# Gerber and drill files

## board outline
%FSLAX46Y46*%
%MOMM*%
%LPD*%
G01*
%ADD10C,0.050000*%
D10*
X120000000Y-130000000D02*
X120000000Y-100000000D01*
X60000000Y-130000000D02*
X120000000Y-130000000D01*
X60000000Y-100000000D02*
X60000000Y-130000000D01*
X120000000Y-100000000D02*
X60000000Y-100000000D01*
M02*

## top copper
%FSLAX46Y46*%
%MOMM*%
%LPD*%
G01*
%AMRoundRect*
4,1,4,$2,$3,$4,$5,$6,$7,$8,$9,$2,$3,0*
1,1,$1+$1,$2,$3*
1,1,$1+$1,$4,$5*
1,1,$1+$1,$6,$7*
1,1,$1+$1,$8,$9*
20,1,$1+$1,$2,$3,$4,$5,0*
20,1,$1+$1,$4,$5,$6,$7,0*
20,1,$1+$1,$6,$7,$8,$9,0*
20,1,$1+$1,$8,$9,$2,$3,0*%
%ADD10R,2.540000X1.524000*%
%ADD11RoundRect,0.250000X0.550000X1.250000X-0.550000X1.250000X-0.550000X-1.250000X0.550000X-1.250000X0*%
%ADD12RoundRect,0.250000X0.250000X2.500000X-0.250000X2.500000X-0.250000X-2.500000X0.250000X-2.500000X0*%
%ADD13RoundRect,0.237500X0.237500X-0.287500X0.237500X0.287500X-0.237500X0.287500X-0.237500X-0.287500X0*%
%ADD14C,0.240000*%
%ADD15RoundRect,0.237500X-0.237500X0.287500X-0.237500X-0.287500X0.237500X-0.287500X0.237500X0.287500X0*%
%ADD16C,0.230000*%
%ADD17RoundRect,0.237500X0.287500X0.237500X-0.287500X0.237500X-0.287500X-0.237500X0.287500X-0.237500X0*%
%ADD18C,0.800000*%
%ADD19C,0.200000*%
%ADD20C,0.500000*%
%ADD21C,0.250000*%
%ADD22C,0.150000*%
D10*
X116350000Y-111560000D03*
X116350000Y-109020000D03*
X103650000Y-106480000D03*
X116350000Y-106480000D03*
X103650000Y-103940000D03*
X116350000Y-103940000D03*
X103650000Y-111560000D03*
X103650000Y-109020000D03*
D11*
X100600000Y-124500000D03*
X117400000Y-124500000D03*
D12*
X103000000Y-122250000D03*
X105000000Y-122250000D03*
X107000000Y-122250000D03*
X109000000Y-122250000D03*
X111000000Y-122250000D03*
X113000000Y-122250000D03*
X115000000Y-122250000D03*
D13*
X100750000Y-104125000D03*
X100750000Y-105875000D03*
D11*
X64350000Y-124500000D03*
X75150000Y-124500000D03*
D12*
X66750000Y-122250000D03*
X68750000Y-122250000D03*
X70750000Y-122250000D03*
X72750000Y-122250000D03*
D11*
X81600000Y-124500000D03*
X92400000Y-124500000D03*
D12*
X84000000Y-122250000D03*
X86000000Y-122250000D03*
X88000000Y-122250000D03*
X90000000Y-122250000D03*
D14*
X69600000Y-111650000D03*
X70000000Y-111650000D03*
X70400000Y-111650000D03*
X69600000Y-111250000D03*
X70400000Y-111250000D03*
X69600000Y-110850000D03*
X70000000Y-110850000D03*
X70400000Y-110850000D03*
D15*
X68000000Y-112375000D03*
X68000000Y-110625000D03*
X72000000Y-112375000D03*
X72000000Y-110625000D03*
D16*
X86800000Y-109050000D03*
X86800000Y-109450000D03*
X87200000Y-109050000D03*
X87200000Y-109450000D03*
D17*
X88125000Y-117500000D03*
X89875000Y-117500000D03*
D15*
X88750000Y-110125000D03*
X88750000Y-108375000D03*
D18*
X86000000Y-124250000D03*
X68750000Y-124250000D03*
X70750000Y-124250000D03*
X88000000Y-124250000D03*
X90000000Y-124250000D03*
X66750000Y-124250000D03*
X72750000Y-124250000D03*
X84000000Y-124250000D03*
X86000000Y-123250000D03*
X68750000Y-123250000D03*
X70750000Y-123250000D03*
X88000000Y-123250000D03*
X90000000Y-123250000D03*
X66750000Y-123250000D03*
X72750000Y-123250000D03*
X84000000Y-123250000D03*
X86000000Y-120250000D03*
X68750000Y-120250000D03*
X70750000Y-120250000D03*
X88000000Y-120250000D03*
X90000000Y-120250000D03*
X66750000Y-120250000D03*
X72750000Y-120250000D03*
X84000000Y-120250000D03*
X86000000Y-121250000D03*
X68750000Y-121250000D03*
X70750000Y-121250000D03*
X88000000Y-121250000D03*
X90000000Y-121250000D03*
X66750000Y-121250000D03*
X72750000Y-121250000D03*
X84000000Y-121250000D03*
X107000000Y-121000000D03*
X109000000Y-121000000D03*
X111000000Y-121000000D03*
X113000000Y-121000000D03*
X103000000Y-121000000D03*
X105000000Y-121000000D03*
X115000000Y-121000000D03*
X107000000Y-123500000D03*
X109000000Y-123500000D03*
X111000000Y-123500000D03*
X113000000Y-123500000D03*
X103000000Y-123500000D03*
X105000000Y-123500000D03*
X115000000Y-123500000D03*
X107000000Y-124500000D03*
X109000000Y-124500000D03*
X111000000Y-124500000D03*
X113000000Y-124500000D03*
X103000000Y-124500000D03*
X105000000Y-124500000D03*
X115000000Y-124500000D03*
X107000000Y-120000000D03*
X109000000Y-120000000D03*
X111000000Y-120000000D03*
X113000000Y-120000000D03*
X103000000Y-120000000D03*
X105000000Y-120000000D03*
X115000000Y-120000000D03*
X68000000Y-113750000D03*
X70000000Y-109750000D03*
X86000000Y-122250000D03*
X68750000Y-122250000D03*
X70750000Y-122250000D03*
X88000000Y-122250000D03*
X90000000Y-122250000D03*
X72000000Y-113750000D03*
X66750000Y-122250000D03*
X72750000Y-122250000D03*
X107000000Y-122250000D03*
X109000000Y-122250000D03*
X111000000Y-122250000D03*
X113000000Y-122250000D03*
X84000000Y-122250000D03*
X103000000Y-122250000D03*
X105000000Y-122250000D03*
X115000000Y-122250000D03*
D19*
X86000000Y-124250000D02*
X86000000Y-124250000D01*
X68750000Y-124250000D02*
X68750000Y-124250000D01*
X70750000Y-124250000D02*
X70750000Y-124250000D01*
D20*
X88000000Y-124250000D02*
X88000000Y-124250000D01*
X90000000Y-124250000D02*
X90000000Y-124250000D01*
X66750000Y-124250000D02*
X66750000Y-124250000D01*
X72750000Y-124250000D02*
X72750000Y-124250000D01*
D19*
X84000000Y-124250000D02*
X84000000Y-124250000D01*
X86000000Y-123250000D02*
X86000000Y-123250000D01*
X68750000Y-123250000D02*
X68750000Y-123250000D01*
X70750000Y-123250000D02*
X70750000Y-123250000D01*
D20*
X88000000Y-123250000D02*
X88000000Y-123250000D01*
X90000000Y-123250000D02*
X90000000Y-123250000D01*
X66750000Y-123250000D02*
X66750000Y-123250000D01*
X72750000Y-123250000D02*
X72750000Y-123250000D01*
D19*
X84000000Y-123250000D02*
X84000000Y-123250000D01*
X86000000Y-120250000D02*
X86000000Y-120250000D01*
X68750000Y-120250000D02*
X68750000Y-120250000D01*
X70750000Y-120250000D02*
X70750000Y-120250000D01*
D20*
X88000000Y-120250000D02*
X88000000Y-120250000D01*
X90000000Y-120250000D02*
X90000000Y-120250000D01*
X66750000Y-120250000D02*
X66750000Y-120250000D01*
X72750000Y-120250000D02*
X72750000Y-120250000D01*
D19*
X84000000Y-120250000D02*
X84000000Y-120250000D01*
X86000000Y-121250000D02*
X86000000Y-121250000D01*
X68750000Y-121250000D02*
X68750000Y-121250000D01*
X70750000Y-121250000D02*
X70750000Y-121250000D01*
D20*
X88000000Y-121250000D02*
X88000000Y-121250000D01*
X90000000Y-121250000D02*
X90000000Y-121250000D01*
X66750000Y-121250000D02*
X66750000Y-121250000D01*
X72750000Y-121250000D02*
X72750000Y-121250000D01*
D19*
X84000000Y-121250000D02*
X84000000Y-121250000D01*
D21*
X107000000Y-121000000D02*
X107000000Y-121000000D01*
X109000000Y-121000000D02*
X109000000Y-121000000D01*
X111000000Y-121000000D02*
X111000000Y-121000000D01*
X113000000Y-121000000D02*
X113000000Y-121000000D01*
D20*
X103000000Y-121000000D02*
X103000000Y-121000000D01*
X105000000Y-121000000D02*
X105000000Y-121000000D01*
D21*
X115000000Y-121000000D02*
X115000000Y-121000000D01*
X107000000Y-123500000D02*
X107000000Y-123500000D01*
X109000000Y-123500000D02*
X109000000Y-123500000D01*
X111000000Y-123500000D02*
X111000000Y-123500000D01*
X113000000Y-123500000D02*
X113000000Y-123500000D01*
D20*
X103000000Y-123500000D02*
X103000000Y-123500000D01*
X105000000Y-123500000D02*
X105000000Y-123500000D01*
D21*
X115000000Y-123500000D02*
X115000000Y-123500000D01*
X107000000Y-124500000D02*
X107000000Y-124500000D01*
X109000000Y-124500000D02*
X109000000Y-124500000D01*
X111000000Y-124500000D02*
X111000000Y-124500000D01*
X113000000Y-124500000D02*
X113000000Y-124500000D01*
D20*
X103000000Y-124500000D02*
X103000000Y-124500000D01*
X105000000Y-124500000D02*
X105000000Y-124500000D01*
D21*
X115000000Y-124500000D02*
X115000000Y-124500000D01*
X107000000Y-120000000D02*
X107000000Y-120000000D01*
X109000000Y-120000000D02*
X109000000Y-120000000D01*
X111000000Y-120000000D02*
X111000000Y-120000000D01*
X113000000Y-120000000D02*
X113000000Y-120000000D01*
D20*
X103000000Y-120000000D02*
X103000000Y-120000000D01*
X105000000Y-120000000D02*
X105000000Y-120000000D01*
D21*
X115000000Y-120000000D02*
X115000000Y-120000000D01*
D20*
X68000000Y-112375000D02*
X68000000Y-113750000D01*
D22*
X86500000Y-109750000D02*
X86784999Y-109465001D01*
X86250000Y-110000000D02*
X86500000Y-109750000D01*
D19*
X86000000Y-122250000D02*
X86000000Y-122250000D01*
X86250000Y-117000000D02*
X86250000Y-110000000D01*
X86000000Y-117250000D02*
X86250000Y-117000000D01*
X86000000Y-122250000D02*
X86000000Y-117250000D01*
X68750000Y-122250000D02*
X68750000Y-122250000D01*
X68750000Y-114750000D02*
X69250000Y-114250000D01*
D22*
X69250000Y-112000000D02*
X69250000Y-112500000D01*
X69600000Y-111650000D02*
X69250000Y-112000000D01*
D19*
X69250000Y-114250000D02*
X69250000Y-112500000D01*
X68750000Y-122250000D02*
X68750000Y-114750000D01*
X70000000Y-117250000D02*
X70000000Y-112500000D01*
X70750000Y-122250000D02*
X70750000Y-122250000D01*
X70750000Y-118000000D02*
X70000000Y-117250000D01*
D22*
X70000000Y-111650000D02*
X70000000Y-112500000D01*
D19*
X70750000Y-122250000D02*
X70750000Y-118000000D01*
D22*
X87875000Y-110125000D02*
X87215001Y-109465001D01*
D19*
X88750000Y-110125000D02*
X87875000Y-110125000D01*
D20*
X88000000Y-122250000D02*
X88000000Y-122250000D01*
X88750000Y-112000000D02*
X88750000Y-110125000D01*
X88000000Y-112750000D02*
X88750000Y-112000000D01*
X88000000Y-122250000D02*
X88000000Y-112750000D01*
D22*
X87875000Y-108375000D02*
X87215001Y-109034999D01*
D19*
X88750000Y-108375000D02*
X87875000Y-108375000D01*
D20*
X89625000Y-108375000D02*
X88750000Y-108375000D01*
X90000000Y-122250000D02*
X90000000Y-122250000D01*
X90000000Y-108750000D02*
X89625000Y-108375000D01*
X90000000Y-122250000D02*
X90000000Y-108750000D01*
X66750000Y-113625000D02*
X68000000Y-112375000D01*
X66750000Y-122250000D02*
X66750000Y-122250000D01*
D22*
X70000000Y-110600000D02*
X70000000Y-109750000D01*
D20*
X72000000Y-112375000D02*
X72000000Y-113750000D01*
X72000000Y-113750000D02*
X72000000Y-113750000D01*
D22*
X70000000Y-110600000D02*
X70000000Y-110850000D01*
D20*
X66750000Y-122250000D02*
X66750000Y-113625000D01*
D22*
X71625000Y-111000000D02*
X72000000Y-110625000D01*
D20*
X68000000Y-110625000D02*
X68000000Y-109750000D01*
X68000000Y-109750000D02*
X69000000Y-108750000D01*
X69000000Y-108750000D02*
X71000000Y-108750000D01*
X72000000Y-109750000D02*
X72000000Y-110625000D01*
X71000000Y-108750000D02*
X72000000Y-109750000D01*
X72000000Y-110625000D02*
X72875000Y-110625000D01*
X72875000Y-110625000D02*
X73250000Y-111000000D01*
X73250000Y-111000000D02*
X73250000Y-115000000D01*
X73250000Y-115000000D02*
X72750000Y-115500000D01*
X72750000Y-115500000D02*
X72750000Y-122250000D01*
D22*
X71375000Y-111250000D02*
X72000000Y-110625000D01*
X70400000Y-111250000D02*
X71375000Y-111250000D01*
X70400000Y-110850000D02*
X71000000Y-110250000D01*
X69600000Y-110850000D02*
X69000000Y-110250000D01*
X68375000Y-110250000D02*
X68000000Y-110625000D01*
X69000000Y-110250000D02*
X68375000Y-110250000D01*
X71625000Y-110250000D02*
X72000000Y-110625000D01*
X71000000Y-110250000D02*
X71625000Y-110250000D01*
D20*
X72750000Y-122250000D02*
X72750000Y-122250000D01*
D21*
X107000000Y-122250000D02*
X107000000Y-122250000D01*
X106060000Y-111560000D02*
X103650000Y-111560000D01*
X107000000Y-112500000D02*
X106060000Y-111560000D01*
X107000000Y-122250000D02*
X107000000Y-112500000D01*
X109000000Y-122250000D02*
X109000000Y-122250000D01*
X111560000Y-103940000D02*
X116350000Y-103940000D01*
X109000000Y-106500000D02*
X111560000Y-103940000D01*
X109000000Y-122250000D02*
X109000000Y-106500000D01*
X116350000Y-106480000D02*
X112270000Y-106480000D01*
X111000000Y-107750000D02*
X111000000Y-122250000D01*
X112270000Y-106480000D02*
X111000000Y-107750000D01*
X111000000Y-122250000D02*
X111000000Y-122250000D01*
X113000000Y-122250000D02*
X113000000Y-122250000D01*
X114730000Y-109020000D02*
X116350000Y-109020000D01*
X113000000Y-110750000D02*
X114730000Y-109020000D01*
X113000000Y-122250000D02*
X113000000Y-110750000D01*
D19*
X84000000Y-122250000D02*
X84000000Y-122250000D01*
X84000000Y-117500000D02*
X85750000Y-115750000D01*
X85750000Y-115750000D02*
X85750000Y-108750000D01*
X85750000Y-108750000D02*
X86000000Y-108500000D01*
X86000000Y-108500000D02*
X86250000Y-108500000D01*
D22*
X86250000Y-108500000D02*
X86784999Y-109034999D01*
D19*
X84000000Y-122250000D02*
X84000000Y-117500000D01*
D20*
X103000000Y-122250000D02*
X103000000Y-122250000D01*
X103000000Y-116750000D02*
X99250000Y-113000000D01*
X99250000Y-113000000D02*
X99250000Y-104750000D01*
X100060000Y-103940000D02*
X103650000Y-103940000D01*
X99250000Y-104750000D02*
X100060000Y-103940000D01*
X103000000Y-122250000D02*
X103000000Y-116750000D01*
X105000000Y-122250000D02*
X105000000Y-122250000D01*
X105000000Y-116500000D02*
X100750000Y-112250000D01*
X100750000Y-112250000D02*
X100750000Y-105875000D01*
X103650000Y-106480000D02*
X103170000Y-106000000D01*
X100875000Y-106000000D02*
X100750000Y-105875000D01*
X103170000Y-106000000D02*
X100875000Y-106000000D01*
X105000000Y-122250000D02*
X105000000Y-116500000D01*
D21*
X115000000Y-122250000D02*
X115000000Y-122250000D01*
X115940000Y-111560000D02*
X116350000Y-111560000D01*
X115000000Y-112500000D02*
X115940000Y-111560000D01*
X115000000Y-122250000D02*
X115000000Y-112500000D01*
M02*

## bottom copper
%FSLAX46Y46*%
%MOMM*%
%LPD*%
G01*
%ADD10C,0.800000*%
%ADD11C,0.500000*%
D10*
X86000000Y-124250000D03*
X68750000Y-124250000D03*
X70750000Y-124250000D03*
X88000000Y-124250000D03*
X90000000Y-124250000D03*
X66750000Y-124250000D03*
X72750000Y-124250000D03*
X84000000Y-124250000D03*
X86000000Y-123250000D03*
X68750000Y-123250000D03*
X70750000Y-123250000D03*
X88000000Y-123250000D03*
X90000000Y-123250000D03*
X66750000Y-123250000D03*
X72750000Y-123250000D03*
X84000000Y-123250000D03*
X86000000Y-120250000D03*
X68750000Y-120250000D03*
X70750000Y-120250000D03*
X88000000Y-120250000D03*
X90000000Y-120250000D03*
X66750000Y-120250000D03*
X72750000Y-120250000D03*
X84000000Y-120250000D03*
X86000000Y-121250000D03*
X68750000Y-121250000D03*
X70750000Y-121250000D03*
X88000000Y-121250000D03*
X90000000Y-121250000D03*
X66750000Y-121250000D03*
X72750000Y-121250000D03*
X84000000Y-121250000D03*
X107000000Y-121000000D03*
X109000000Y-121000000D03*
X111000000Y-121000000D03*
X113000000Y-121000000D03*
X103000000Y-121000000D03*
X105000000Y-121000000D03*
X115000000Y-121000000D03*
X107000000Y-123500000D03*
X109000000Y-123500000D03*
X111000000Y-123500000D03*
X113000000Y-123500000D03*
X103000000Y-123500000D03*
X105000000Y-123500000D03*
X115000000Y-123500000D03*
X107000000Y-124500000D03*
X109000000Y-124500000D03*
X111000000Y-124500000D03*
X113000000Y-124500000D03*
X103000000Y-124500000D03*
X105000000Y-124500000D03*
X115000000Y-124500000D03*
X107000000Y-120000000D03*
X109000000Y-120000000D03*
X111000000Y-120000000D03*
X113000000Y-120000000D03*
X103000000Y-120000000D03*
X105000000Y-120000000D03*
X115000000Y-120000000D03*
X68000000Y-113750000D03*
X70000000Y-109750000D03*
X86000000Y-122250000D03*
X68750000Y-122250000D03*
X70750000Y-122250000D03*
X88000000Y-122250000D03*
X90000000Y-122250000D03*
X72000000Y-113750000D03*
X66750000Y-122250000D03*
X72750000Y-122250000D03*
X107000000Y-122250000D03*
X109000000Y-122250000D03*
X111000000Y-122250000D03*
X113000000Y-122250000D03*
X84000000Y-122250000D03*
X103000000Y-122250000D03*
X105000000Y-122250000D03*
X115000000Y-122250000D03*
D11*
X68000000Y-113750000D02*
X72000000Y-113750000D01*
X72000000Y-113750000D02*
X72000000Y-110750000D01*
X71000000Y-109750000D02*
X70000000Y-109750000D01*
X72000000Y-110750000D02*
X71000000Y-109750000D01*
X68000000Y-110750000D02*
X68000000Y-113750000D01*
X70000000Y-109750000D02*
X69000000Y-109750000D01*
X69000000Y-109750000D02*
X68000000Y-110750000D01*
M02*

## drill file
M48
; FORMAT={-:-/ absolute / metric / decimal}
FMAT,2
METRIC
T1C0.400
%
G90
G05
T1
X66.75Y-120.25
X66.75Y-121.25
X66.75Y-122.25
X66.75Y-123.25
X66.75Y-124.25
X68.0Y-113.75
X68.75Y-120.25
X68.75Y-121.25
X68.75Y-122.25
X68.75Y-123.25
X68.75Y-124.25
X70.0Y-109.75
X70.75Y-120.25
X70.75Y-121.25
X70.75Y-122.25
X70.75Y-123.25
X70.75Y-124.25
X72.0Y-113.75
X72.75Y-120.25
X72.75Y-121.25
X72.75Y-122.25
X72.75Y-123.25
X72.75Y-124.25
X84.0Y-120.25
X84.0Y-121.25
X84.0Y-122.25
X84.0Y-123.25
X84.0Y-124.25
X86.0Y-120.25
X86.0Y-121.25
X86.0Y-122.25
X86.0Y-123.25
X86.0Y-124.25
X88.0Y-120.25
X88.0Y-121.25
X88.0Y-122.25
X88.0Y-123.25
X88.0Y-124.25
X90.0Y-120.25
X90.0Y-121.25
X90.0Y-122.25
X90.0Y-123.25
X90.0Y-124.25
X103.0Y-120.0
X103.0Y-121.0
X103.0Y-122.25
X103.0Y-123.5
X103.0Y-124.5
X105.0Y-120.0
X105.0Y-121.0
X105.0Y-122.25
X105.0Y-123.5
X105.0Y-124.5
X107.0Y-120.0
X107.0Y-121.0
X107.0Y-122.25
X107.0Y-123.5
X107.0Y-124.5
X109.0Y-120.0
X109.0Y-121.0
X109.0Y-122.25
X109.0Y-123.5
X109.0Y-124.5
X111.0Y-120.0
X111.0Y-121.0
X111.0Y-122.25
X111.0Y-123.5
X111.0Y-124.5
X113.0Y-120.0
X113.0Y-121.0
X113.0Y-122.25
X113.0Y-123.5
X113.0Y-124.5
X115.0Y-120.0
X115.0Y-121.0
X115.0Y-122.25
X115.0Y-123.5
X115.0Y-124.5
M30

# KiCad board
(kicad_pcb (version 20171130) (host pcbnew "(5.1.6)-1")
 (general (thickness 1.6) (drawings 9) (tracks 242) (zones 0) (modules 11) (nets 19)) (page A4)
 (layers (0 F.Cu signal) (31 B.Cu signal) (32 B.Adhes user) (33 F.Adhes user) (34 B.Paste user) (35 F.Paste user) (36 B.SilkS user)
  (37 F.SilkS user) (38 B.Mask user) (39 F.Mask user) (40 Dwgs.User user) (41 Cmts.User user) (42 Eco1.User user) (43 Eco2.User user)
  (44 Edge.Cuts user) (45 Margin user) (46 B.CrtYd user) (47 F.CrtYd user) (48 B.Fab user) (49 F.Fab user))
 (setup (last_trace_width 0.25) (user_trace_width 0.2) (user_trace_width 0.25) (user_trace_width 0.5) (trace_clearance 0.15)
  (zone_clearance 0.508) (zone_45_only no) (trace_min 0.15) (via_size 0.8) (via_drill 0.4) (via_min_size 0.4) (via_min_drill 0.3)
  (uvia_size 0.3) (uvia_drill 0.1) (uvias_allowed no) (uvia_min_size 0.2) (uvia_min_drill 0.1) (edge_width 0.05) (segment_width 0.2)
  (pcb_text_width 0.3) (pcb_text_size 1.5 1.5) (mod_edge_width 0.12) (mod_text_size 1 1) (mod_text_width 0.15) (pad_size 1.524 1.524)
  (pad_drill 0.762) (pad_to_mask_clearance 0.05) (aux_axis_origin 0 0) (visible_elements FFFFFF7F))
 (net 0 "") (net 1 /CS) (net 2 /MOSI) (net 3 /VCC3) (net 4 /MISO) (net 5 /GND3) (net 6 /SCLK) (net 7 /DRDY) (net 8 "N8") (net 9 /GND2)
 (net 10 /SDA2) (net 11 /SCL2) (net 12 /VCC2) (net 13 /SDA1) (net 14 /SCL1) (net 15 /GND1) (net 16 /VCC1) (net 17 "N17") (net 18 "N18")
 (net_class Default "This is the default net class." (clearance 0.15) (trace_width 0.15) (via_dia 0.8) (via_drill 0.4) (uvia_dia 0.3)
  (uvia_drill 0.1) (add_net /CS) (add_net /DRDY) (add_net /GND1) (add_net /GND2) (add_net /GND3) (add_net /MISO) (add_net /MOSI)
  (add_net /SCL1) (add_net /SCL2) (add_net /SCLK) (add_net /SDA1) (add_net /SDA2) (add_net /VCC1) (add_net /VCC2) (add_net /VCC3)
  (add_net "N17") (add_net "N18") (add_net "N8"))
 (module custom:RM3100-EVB (layer F.Cu) (at 110 107.75)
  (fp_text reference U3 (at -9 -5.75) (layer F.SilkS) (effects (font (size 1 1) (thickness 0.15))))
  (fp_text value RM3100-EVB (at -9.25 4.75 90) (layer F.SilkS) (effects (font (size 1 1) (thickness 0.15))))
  (pad 8 smd rect (at 6.35 3.81) (size 2.54 1.524) (layers F.Cu F.Paste F.Mask) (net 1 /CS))
  (pad 7 smd rect (at 6.35 1.27) (size 2.54 1.524) (layers F.Cu F.Paste F.Mask) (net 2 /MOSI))
  (pad 2 smd rect (at -6.35 -1.27) (size 2.54 1.524) (layers F.Cu F.Paste F.Mask) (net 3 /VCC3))
  (pad 6 smd rect (at 6.35 -1.27) (size 2.54 1.524) (layers F.Cu F.Paste F.Mask) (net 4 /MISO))
  (pad 1 smd rect (at -6.35 -3.81) (size 2.54 1.524) (layers F.Cu F.Paste F.Mask) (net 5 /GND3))
  (pad 5 smd rect (at 6.35 -3.81) (size 2.54 1.524) (layers F.Cu F.Paste F.Mask) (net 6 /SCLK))
  (pad 4 smd rect (at -6.35 3.81) (size 2.54 1.524) (layers F.Cu F.Paste F.Mask) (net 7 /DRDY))
  (pad 3 smd rect (at -6.35 1.27) (size 2.54 1.524) (layers F.Cu F.Paste F.Mask) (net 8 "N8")))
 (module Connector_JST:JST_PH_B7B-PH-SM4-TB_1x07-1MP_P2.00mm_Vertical (layer F.Cu) (at 109 122.75 180)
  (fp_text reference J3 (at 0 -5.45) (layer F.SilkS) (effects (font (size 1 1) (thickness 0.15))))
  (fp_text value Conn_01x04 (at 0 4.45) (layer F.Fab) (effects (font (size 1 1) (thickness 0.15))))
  (pad MP smd roundrect (at 8.4 -1.75 180) (size 1.6 3) (layers F.Cu F.Paste F.Mask) (roundrect_rratio 0.15625))
  (pad MP smd roundrect (at -8.4 -1.75 180) (size 1.6 3) (layers F.Cu F.Paste F.Mask) (roundrect_rratio 0.15625))
  (pad 7 smd roundrect (at 6 0.5 180) (size 1 5.5) (layers F.Cu F.Paste F.Mask) (roundrect_rratio 0.25) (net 5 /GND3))
  (pad 6 smd roundrect (at 4 0.5 180) (size 1 5.5) (layers F.Cu F.Paste F.Mask) (roundrect_rratio 0.25) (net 3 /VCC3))
  (pad 5 smd roundrect (at 2 0.5 180) (size 1 5.5) (layers F.Cu F.Paste F.Mask) (roundrect_rratio 0.25) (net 7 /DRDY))
  (pad 4 smd roundrect (at 0 0.5 180) (size 1 5.5) (layers F.Cu F.Paste F.Mask) (roundrect_rratio 0.25) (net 6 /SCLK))
  (pad 3 smd roundrect (at -2 0.5 180) (size 1 5.5) (layers F.Cu F.Paste F.Mask) (roundrect_rratio 0.25) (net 4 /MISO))
  (pad 2 smd roundrect (at -4 0.5 180) (size 1 5.5) (layers F.Cu F.Paste F.Mask) (roundrect_rratio 0.25) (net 2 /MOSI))
  (pad 1 smd roundrect (at -6 0.5 180) (size 1 5.5) (layers F.Cu F.Paste F.Mask) (roundrect_rratio 0.25) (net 1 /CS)))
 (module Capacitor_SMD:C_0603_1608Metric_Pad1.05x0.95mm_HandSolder (layer F.Cu) (at 100.75 105 90)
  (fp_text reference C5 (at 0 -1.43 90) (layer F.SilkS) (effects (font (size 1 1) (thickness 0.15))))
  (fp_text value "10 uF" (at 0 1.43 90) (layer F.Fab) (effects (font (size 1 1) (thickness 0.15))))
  (pad 2 smd roundrect (at 0.875 0 90) (size 1.05 0.95) (layers F.Cu F.Paste F.Mask) (roundrect_rratio 0.25) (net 5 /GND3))
  (pad 1 smd roundrect (at -0.875 0 90) (size 1.05 0.95) (layers F.Cu F.Paste F.Mask) (roundrect_rratio 0.25) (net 3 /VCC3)))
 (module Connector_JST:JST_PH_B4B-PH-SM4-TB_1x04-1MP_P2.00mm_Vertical (layer F.Cu) (at 69.75 122.75 180)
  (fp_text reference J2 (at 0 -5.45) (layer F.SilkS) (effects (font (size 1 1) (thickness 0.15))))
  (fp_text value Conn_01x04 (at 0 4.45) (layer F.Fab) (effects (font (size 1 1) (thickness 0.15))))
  (pad MP smd roundrect (at 5.4 -1.75 180) (size 1.6 3) (layers F.Cu F.Paste F.Mask) (roundrect_rratio 0.15625))
  (pad MP smd roundrect (at -5.4 -1.75 180) (size 1.6 3) (layers F.Cu F.Paste F.Mask) (roundrect_rratio 0.15625))
  (pad 4 smd roundrect (at 3 0.5 180) (size 1 5.5) (layers F.Cu F.Paste F.Mask) (roundrect_rratio 0.25) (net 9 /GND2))
  (pad 3 smd roundrect (at 1 0.5 180) (size 1 5.5) (layers F.Cu F.Paste F.Mask) (roundrect_rratio 0.25) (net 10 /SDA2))
  (pad 2 smd roundrect (at -1 0.5 180) (size 1 5.5) (layers F.Cu F.Paste F.Mask) (roundrect_rratio 0.25) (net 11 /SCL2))
  (pad 1 smd roundrect (at -3 0.5 180) (size 1 5.5) (layers F.Cu F.Paste F.Mask) (roundrect_rratio 0.25) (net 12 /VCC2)))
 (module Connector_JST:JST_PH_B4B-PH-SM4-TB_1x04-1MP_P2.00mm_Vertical (layer F.Cu) (at 87 122.75 180)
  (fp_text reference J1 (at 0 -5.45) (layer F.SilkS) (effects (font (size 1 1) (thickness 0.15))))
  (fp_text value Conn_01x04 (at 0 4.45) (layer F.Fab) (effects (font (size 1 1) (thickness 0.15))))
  (pad MP smd roundrect (at 5.4 -1.75 180) (size 1.6 3) (layers F.Cu F.Paste F.Mask) (roundrect_rratio 0.15625))
  (pad MP smd roundrect (at -5.4 -1.75 180) (size 1.6 3) (layers F.Cu F.Paste F.Mask) (roundrect_rratio 0.15625))
  (pad 4 smd roundrect (at 3 0.5 180) (size 1 5.5) (layers F.Cu F.Paste F.Mask) (roundrect_rratio 0.25) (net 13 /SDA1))
  (pad 3 smd roundrect (at 1 0.5 180) (size 1 5.5) (layers F.Cu F.Paste F.Mask) (roundrect_rratio 0.25) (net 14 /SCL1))
  (pad 2 smd roundrect (at -1 0.5 180) (size 1 5.5) (layers F.Cu F.Paste F.Mask) (roundrect_rratio 0.25) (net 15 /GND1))
  (pad 1 smd roundrect (at -3 0.5 180) (size 1 5.5) (layers F.Cu F.Paste F.Mask) (roundrect_rratio 0.25) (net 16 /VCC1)))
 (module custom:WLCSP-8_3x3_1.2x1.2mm (layer F.Cu) (at 70 111.25 270)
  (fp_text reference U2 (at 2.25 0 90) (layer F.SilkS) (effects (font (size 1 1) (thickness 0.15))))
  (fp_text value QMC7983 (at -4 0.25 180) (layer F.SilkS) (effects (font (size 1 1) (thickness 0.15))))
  (pad C3 smd circle (at 0.4 0.4 270) (size 0.24 0.24) (layers F.Cu F.Paste F.Mask) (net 10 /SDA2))
  (pad B3 smd circle (at 0.4 0 270) (size 0.24 0.24) (layers F.Cu F.Paste F.Mask) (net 11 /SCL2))
  (pad A3 smd circle (at 0.4 -0.4 270) (size 0.24 0.24) (layers F.Cu F.Paste F.Mask) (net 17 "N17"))
  (pad C2 smd circle (at 0 0.4 270) (size 0.24 0.24) (layers F.Cu F.Paste F.Mask) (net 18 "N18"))
  (pad A2 smd circle (at 0 -0.4 270) (size 0.24 0.24) (layers F.Cu F.Paste F.Mask) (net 12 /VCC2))
  (pad C1 smd circle (at -0.4 0.4 270) (size 0.24 0.24) (layers F.Cu F.Paste F.Mask) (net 12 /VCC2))
  (pad B1 smd circle (at -0.4 0 270) (size 0.24 0.24) (layers F.Cu F.Paste F.Mask) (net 9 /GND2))
  (pad A1 smd circle (at -0.4 -0.4 270) (size 0.24 0.24) (layers F.Cu F.Paste F.Mask) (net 12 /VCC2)))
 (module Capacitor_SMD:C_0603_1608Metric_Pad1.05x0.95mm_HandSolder (layer F.Cu) (at 68 111.5 270)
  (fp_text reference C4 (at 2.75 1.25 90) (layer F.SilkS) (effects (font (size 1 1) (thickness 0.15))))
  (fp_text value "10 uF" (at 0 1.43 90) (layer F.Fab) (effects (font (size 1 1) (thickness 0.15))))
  (pad 2 smd roundrect (at 0.875 0 270) (size 1.05 0.95) (layers F.Cu F.Paste F.Mask) (roundrect_rratio 0.25) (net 9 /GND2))
  (pad 1 smd roundrect (at -0.875 0 270) (size 1.05 0.95) (layers F.Cu F.Paste F.Mask) (roundrect_rratio 0.25) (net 12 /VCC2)))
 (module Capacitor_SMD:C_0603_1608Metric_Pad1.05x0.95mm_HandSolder (layer F.Cu) (at 72 111.5 270)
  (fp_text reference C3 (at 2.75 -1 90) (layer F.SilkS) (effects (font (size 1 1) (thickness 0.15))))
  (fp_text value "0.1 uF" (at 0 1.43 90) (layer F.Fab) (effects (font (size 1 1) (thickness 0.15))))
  (pad 2 smd roundrect (at 0.875 0 270) (size 1.05 0.95) (layers F.Cu F.Paste F.Mask) (roundrect_rratio 0.25) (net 9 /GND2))
  (pad 1 smd roundrect (at -0.875 0 270) (size 1.05 0.95) (layers F.Cu F.Paste F.Mask) (roundrect_rratio 0.25) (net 12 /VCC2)))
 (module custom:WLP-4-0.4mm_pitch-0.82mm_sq (layer F.Cu) (at 87 109.25 180)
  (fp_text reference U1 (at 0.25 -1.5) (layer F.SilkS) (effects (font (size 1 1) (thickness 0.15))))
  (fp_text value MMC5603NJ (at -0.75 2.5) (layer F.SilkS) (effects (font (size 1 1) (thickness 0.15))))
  (pad B2 smd circle (at 0.2 0.2 180) (size 0.23 0.23) (layers F.Cu F.Paste F.Mask) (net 13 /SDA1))
  (pad A2 smd circle (at 0.2 -0.2 180) (size 0.23 0.23) (layers F.Cu F.Paste F.Mask) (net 14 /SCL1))
  (pad B1 smd circle (at -0.2 0.2 180) (size 0.23 0.23) (layers F.Cu F.Paste F.Mask) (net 16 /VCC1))
  (pad A1 smd circle (at -0.2 -0.2 180) (size 0.23 0.23) (layers F.Cu F.Paste F.Mask) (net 15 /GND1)))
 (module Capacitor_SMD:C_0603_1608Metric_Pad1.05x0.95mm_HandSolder (layer F.Cu) (at 89 117.5 180)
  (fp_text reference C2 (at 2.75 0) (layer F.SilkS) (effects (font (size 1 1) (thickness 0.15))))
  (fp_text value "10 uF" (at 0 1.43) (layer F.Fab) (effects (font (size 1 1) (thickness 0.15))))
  (pad 2 smd roundrect (at 0.875 0 180) (size 1.05 0.95) (layers F.Cu F.Paste F.Mask) (roundrect_rratio 0.25) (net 15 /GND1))
  (pad 1 smd roundrect (at -0.875 0 180) (size 1.05 0.95) (layers F.Cu F.Paste F.Mask) (roundrect_rratio 0.25) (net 16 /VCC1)))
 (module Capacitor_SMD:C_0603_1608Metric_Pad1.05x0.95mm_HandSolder (layer F.Cu) (at 88.75 109.25 270)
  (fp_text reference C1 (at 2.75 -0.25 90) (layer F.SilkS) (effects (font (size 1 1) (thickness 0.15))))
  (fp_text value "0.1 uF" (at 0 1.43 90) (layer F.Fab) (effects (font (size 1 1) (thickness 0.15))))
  (pad 2 smd roundrect (at 0.875 0 270) (size 1.05 0.95) (layers F.Cu F.Paste F.Mask) (roundrect_rratio 0.25) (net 15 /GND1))
  (pad 1 smd roundrect (at -0.875 0 270) (size 1.05 0.95) (layers F.Cu F.Paste F.Mask) (roundrect_rratio 0.25) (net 16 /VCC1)))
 (gr_line (start 120 130) (end 120 100) (layer Edge.Cuts) (width 0.05))
 (gr_line (start 60 130) (end 120 130) (layer Edge.Cuts) (width 0.05))
 (gr_line (start 60 100) (end 60 130) (layer Edge.Cuts) (width 0.05))
 (gr_line (start 120 100) (end 60 100) (layer Edge.Cuts) (width 0.05))
 (via (at 86 124.25) (size 0.8) (drill 0.4) (layers F.Cu B.Cu) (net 14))
 (segment (start 86 124.25) (end 86 124.25) (width 0.2) (layer F.Cu) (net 14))
 (via (at 68.75 124.25) (size 0.8) (drill 0.4) (layers F.Cu B.Cu) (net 10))
 (segment (start 68.75 124.25) (end 68.75 124.25) (width 0.2) (layer F.Cu) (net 10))
 (segment (start 70.75 124.25) (end 70.75 124.25) (width 0.2) (layer F.Cu) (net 11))
 (via (at 70.75 124.25) (size 0.8) (drill 0.4) (layers F.Cu B.Cu) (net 11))
 (via (at 88 124.25) (size 0.8) (drill 0.4) (layers F.Cu B.Cu) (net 15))
 (segment (start 88 124.25) (end 88 124.25) (width 0.5) (layer F.Cu) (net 15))
 (via (at 90 124.25) (size 0.8) (drill 0.4) (layers F.Cu B.Cu) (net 16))
 (segment (start 90 124.25) (end 90 124.25) (width 0.5) (layer F.Cu) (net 16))
 (via (at 66.75 124.25) (size 0.8) (drill 0.4) (layers F.Cu B.Cu) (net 9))
 (segment (start 66.75 124.25) (end 66.75 124.25) (width 0.5) (layer F.Cu) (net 9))
 (segment (start 72.75 124.25) (end 72.75 124.25) (width 0.5) (layer F.Cu) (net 12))
 (via (at 72.75 124.25) (size 0.8) (drill 0.4) (layers F.Cu B.Cu) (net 12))
 (via (at 84 124.25) (size 0.8) (drill 0.4) (layers F.Cu B.Cu) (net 13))
 (segment (start 84 124.25) (end 84 124.25) (width 0.2) (layer F.Cu) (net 13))
 (via (at 86 123.25) (size 0.8) (drill 0.4) (layers F.Cu B.Cu) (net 14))
 (segment (start 86 123.25) (end 86 123.25) (width 0.2) (layer F.Cu) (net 14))
 (via (at 68.75 123.25) (size 0.8) (drill 0.4) (layers F.Cu B.Cu) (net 10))
 (segment (start 68.75 123.25) (end 68.75 123.25) (width 0.2) (layer F.Cu) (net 10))
 (segment (start 70.75 123.25) (end 70.75 123.25) (width 0.2) (layer F.Cu) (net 11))
 (via (at 70.75 123.25) (size 0.8) (drill 0.4) (layers F.Cu B.Cu) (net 11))
 (via (at 88 123.25) (size 0.8) (drill 0.4) (layers F.Cu B.Cu) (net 15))
 (segment (start 88 123.25) (end 88 123.25) (width 0.5) (layer F.Cu) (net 15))
 (via (at 90 123.25) (size 0.8) (drill 0.4) (layers F.Cu B.Cu) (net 16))
 (segment (start 90 123.25) (end 90 123.25) (width 0.5) (layer F.Cu) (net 16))
 (via (at 66.75 123.25) (size 0.8) (drill 0.4) (layers F.Cu B.Cu) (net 9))
 (segment (start 66.75 123.25) (end 66.75 123.25) (width 0.5) (layer F.Cu) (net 9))
 (segment (start 72.75 123.25) (end 72.75 123.25) (width 0.5) (layer F.Cu) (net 12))
 (via (at 72.75 123.25) (size 0.8) (drill 0.4) (layers F.Cu B.Cu) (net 12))
 (via (at 84 123.25) (size 0.8) (drill 0.4) (layers F.Cu B.Cu) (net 13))
 (segment (start 84 123.25) (end 84 123.25) (width 0.2) (layer F.Cu) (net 13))
 (via (at 86 120.25) (size 0.8) (drill 0.4) (layers F.Cu B.Cu) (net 14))
 (segment (start 86 120.25) (end 86 120.25) (width 0.2) (layer F.Cu) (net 14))
 (via (at 68.75 120.25) (size 0.8) (drill 0.4) (layers F.Cu B.Cu) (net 10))
 (segment (start 68.75 120.25) (end 68.75 120.25) (width 0.2) (layer F.Cu) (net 10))
 (segment (start 70.75 120.25) (end 70.75 120.25) (width 0.2) (layer F.Cu) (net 11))
 (via (at 70.75 120.25) (size 0.8) (drill 0.4) (layers F.Cu B.Cu) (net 11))
 (via (at 88 120.25) (size 0.8) (drill 0.4) (layers F.Cu B.Cu) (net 15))
 (segment (start 88 120.25) (end 88 120.25) (width 0.5) (layer F.Cu) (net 15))
 (via (at 90 120.25) (size 0.8) (drill 0.4) (layers F.Cu B.Cu) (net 16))
 (segment (start 90 120.25) (end 90 120.25) (width 0.5) (layer F.Cu) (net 16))
 (via (at 66.75 120.25) (size 0.8) (drill 0.4) (layers F.Cu B.Cu) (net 9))
 (segment (start 66.75 120.25) (end 66.75 120.25) (width 0.5) (layer F.Cu) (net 9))
 (segment (start 72.75 120.25) (end 72.75 120.25) (width 0.5) (layer F.Cu) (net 12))
 (via (at 72.75 120.25) (size 0.8) (drill 0.4) (layers F.Cu B.Cu) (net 12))
 (via (at 84 120.25) (size 0.8) (drill 0.4) (layers F.Cu B.Cu) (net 13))
 (segment (start 84 120.25) (end 84 120.25) (width 0.2) (layer F.Cu) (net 13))
 (via (at 86 121.25) (size 0.8) (drill 0.4) (layers F.Cu B.Cu) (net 14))
 (segment (start 86 121.25) (end 86 121.25) (width 0.2) (layer F.Cu) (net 14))
 (via (at 68.75 121.25) (size 0.8) (drill 0.4) (layers F.Cu B.Cu) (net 10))
 (segment (start 68.75 121.25) (end 68.75 121.25) (width 0.2) (layer F.Cu) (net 10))
 (segment (start 70.75 121.25) (end 70.75 121.25) (width 0.2) (layer F.Cu) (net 11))
 (via (at 70.75 121.25) (size 0.8) (drill 0.4) (layers F.Cu B.Cu) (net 11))
 (via (at 88 121.25) (size 0.8) (drill 0.4) (layers F.Cu B.Cu) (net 15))
 (segment (start 88 121.25) (end 88 121.25) (width 0.5) (layer F.Cu) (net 15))
 (via (at 90 121.25) (size 0.8) (drill 0.4) (layers F.Cu B.Cu) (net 16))
 (segment (start 90 121.25) (end 90 121.25) (width 0.5) (layer F.Cu) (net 16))
 (via (at 66.75 121.25) (size 0.8) (drill 0.4) (layers F.Cu B.Cu) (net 9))
 (segment (start 66.75 121.25) (end 66.75 121.25) (width 0.5) (layer F.Cu) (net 9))
 (segment (start 72.75 121.25) (end 72.75 121.25) (width 0.5) (layer F.Cu) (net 12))
 (via (at 72.75 121.25) (size 0.8) (drill 0.4) (layers F.Cu B.Cu) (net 12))
 (via (at 84 121.25) (size 0.8) (drill 0.4) (layers F.Cu B.Cu) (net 13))
 (segment (start 84 121.25) (end 84 121.25) (width 0.2) (layer F.Cu) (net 13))
 (via (at 107 121) (size 0.8) (drill 0.4) (layers F.Cu B.Cu) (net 7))
 (segment (start 107 121) (end 107 121) (width 0.25) (layer F.Cu) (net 7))
 (via (at 109 121) (size 0.8) (drill 0.4) (layers F.Cu B.Cu) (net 6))
 (segment (start 109 121) (end 109 121) (width 0.25) (layer F.Cu) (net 6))
 (via (at 111 121) (size 0.8) (drill 0.4) (layers F.Cu B.Cu) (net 4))
 (segment (start 111 121) (end 111 121) (width 0.25) (layer F.Cu) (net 4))
 (segment (start 113 121) (end 113 121) (width 0.25) (layer F.Cu) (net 2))
 (via (at 113 121) (size 0.8) (drill 0.4) (layers F.Cu B.Cu) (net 2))
 (via (at 103 121) (size 0.8) (drill 0.4) (layers F.Cu B.Cu) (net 5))
 (segment (start 103 121) (end 103 121) (width 0.5) (layer F.Cu) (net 5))
 (segment (start 105 121) (end 105 121) (width 0.5) (layer F.Cu) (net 3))
 (via (at 105 121) (size 0.8) (drill 0.4) (layers F.Cu B.Cu) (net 3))
 (segment (start 115 121) (end 115 121) (width 0.25) (layer F.Cu) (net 1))
 (via (at 115 121) (size 0.8) (drill 0.4) (layers F.Cu B.Cu) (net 1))
 (via (at 107 123.5) (size 0.8) (drill 0.4) (layers F.Cu B.Cu) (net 7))
 (segment (start 107 123.5) (end 107 123.5) (width 0.25) (layer F.Cu) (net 7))
 (via (at 109 123.5) (size 0.8) (drill 0.4) (layers F.Cu B.Cu) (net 6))
 (segment (start 109 123.5) (end 109 123.5) (width 0.25) (layer F.Cu) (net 6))
 (via (at 111 123.5) (size 0.8) (drill 0.4) (layers F.Cu B.Cu) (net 4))
 (segment (start 111 123.5) (end 111 123.5) (width 0.25) (layer F.Cu) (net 4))
 (segment (start 113 123.5) (end 113 123.5) (width 0.25) (layer F.Cu) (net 2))
 (via (at 113 123.5) (size 0.8) (drill 0.4) (layers F.Cu B.Cu) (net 2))
 (via (at 103 123.5) (size 0.8) (drill 0.4) (layers F.Cu B.Cu) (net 5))
 (segment (start 103 123.5) (end 103 123.5) (width 0.5) (layer F.Cu) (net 5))
 (segment (start 105 123.5) (end 105 123.5) (width 0.5) (layer F.Cu) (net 3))
 (via (at 105 123.5) (size 0.8) (drill 0.4) (layers F.Cu B.Cu) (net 3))
 (segment (start 115 123.5) (end 115 123.5) (width 0.25) (layer F.Cu) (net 1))
 (via (at 115 123.5) (size 0.8) (drill 0.4) (layers F.Cu B.Cu) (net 1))
 (via (at 107 124.5) (size 0.8) (drill 0.4) (layers F.Cu B.Cu) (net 7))
 (segment (start 107 124.5) (end 107 124.5) (width 0.25) (layer F.Cu) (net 7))
 (via (at 109 124.5) (size 0.8) (drill 0.4) (layers F.Cu B.Cu) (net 6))
 (segment (start 109 124.5) (end 109 124.5) (width 0.25) (layer F.Cu) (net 6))
 (via (at 111 124.5) (size 0.8) (drill 0.4) (layers F.Cu B.Cu) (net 4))
 (segment (start 111 124.5) (end 111 124.5) (width 0.25) (layer F.Cu) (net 4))
 (segment (start 113 124.5) (end 113 124.5) (width 0.25) (layer F.Cu) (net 2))
 (via (at 113 124.5) (size 0.8) (drill 0.4) (layers F.Cu B.Cu) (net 2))
 (via (at 103 124.5) (size 0.8) (drill 0.4) (layers F.Cu B.Cu) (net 5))
 (segment (start 103 124.5) (end 103 124.5) (width 0.5) (layer F.Cu) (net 5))
 (segment (start 105 124.5) (end 105 124.5) (width 0.5) (layer F.Cu) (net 3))
 (via (at 105 124.5) (size 0.8) (drill 0.4) (layers F.Cu B.Cu) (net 3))
 (segment (start 115 124.5) (end 115 124.5) (width 0.25) (layer F.Cu) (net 1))
 (via (at 115 124.5) (size 0.8) (drill 0.4) (layers F.Cu B.Cu) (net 1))
 (via (at 107 120) (size 0.8) (drill 0.4) (layers F.Cu B.Cu) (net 7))
 (segment (start 107 120) (end 107 120) (width 0.25) (layer F.Cu) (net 7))
 (via (at 109 120) (size 0.8) (drill 0.4) (layers F.Cu B.Cu) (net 6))
 (segment (start 109 120) (end 109 120) (width 0.25) (layer F.Cu) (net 6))
 (via (at 111 120) (size 0.8) (drill 0.4) (layers F.Cu B.Cu) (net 4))
 (segment (start 111 120) (end 111 120) (width 0.25) (layer F.Cu) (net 4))
 (segment (start 113 120) (end 113 120) (width 0.25) (layer F.Cu) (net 2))
 (via (at 113 120) (size 0.8) (drill 0.4) (layers F.Cu B.Cu) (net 2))
 (via (at 103 120) (size 0.8) (drill 0.4) (layers F.Cu B.Cu) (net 5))
 (segment (start 103 120) (end 103 120) (width 0.5) (layer F.Cu) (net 5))
 (segment (start 105 120) (end 105 120) (width 0.5) (layer F.Cu) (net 3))
 (via (at 105 120) (size 0.8) (drill 0.4) (layers F.Cu B.Cu) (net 3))
 (segment (start 115 120) (end 115 120) (width 0.25) (layer F.Cu) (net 1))
 (via (at 115 120) (size 0.8) (drill 0.4) (layers F.Cu B.Cu) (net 1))
 (via (at 68 113.75) (size 0.8) (drill 0.4) (layers F.Cu B.Cu) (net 9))
 (segment (start 68 112.375) (end 68 113.75) (width 0.5) (layer F.Cu) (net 9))
 (via (at 70 109.75) (size 0.8) (drill 0.4) (layers F.Cu B.Cu) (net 9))
 (segment (start 86.5 109.75) (end 86.784999 109.465001) (width 0.15) (layer F.Cu) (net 14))
 (segment (start 86.25 110) (end 86.5 109.75) (width 0.15) (layer F.Cu) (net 14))
 (segment (start 86 122.25) (end 86 122.25) (width 0.2) (layer F.Cu) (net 14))
 (segment (start 86.25 117) (end 86.25 110) (width 0.2) (layer F.Cu) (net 14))
 (segment (start 86 117.25) (end 86.25 117) (width 0.2) (layer F.Cu) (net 14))
 (segment (start 86 122.25) (end 86 117.25) (width 0.2) (layer F.Cu) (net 14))
 (via (at 86 122.25) (size 0.8) (drill 0.4) (layers F.Cu B.Cu) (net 14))
 (segment (start 68.75 122.25) (end 68.75 122.25) (width 0.2) (layer F.Cu) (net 10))
 (segment (start 68.75 114.75) (end 69.25 114.25) (width 0.2) (layer F.Cu) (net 10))
 (segment (start 69.25 112) (end 69.25 112.5) (width 0.15) (layer F.Cu) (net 10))
 (segment (start 69.6 111.65) (end 69.25 112) (width 0.15) (layer F.Cu) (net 10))
 (segment (start 69.25 114.25) (end 69.25 112.5) (width 0.2) (layer F.Cu) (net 10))
 (segment (start 68.75 122.25) (end 68.75 114.75) (width 0.2) (layer F.Cu) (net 10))
 (via (at 68.75 122.25) (size 0.8) (drill 0.4) (layers F.Cu B.Cu) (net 10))
 (segment (start 70 117.25) (end 70 112.5) (width 0.2) (layer F.Cu) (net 11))
 (segment (start 70.75 122.25) (end 70.75 122.25) (width 0.2) (layer F.Cu) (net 11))
 (segment (start 70.75 118) (end 70 117.25) (width 0.2) (layer F.Cu) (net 11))
 (segment (start 70 111.65) (end 70 112.5) (width 0.15) (layer F.Cu) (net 11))
 (segment (start 70.75 122.25) (end 70.75 118) (width 0.2) (layer F.Cu) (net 11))
 (via (at 70.75 122.25) (size 0.8) (drill 0.4) (layers F.Cu B.Cu) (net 11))
 (segment (start 87.875 110.125) (end 87.215001 109.465001) (width 0.15) (layer F.Cu) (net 15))
 (segment (start 88.75 110.125) (end 87.875 110.125) (width 0.2) (layer F.Cu) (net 15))
 (segment (start 88 122.25) (end 88 122.25) (width 0.5) (layer F.Cu) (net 15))
 (segment (start 88.75 112) (end 88.75 110.125) (width 0.5) (layer F.Cu) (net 15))
 (segment (start 88 112.75) (end 88.75 112) (width 0.5) (layer F.Cu) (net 15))
 (segment (start 88 122.25) (end 88 112.75) (width 0.5) (layer F.Cu) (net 15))
 (via (at 88 122.25) (size 0.8) (drill 0.4) (layers F.Cu B.Cu) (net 15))
 (segment (start 87.875 108.375) (end 87.215001 109.034999) (width 0.15) (layer F.Cu) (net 16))
 (segment (start 88.75 108.375) (end 87.875 108.375) (width 0.2) (layer F.Cu) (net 16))
 (segment (start 89.625 108.375) (end 88.75 108.375) (width 0.5) (layer F.Cu) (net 16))
 (segment (start 90 122.25) (end 90 122.25) (width 0.5) (layer F.Cu) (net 16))
 (segment (start 90 108.75) (end 89.625 108.375) (width 0.5) (layer F.Cu) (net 16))
 (segment (start 90 122.25) (end 90 108.75) (width 0.5) (layer F.Cu) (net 16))
 (via (at 90 122.25) (size 0.8) (drill 0.4) (layers F.Cu B.Cu) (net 16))
 (segment (start 66.75 113.625) (end 68 112.375) (width 0.5) (layer F.Cu) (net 9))
 (segment (start 66.75 122.25) (end 66.75 122.25) (width 0.5) (layer F.Cu) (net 9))
 (segment (start 70 110.6) (end 70 109.75) (width 0.15) (layer F.Cu) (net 9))
 (segment (start 72 112.375) (end 72 113.75) (width 0.5) (layer F.Cu) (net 9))
 (segment (start 72 113.75) (end 72 113.75) (width 0.5) (layer F.Cu) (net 9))
 (via (at 72 113.75) (size 0.8) (drill 0.4) (layers F.Cu B.Cu) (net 9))
 (segment (start 68 113.75) (end 72 113.75) (width 0.5) (layer B.Cu) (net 9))
 (segment (start 72 113.75) (end 72 110.75) (width 0.5) (layer B.Cu) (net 9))
 (segment (start 71 109.75) (end 70 109.75) (width 0.5) (layer B.Cu) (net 9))
 (segment (start 72 110.75) (end 71 109.75) (width 0.5) (layer B.Cu) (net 9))
 (segment (start 68 110.75) (end 68 113.75) (width 0.5) (layer B.Cu) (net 9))
 (segment (start 70 109.75) (end 69 109.75) (width 0.5) (layer B.Cu) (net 9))
 (segment (start 69 109.75) (end 68 110.75) (width 0.5) (layer B.Cu) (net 9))
 (segment (start 70 110.6) (end 70 110.85) (width 0.15) (layer F.Cu) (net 9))
 (segment (start 66.75 122.25) (end 66.75 113.625) (width 0.5) (layer F.Cu) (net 9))
 (via (at 66.75 122.25) (size 0.8) (drill 0.4) (layers F.Cu B.Cu) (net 9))
 (segment (start 71.625 111) (end 72 110.625) (width 0.15) (layer F.Cu) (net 12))
 (segment (start 68 110.625) (end 68 109.75) (width 0.5) (layer F.Cu) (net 12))
 (segment (start 68 109.75) (end 69 108.75) (width 0.5) (layer F.Cu) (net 12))
 (segment (start 69 108.75) (end 71 108.75) (width 0.5) (layer F.Cu) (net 12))
 (segment (start 72 109.75) (end 72 110.625) (width 0.5) (layer F.Cu) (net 12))
 (segment (start 71 108.75) (end 72 109.75) (width 0.5) (layer F.Cu) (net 12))
 (segment (start 72 110.625) (end 72.875 110.625) (width 0.5) (layer F.Cu) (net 12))
 (segment (start 72.875 110.625) (end 73.25 111) (width 0.5) (layer F.Cu) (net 12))
 (segment (start 73.25 111) (end 73.25 115) (width 0.5) (layer F.Cu) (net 12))
 (segment (start 73.25 115) (end 72.75 115.5) (width 0.5) (layer F.Cu) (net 12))
 (segment (start 72.75 115.5) (end 72.75 122.25) (width 0.5) (layer F.Cu) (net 12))
 (segment (start 71.375 111.25) (end 72 110.625) (width 0.15) (layer F.Cu) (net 12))
 (segment (start 70.4 111.25) (end 71.375 111.25) (width 0.15) (layer F.Cu) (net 12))
 (segment (start 70.4 110.85) (end 71 110.25) (width 0.15) (layer F.Cu) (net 12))
 (segment (start 69.6 110.85) (end 69 110.25) (width 0.15) (layer F.Cu) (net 12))
 (segment (start 68.375 110.25) (end 68 110.625) (width 0.15) (layer F.Cu) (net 12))
 (segment (start 69 110.25) (end 68.375 110.25) (width 0.15) (layer F.Cu) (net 12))
 (segment (start 71.625 110.25) (end 72 110.625) (width 0.15) (layer F.Cu) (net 12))
 (segment (start 71 110.25) (end 71.625 110.25) (width 0.15) (layer F.Cu) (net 12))
 (segment (start 72.75 122.25) (end 72.75 122.25) (width 0.5) (layer F.Cu) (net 12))
 (via (at 72.75 122.25) (size 0.8) (drill 0.4) (layers F.Cu B.Cu) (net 12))
 (segment (start 107 122.25) (end 107 122.25) (width 0.25) (layer F.Cu) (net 7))
 (segment (start 106.06 111.56) (end 103.65 111.56) (width 0.25) (layer F.Cu) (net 7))
 (segment (start 107 112.5) (end 106.06 111.56) (width 0.25) (layer F.Cu) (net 7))
 (segment (start 107 122.25) (end 107 112.5) (width 0.25) (layer F.Cu) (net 7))
 (via (at 107 122.25) (size 0.8) (drill 0.4) (layers F.Cu B.Cu) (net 7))
 (segment (start 109 122.25) (end 109 122.25) (width 0.25) (layer F.Cu) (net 6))
 (segment (start 111.56 103.94) (end 116.35 103.94) (width 0.25) (layer F.Cu) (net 6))
 (segment (start 109 106.5) (end 111.56 103.94) (width 0.25) (layer F.Cu) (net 6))
 (segment (start 109 122.25) (end 109 106.5) (width 0.25) (layer F.Cu) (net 6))
 (via (at 109 122.25) (size 0.8) (drill 0.4) (layers F.Cu B.Cu) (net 6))
 (segment (start 116.35 106.48) (end 112.27 106.48) (width 0.25) (layer F.Cu) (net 4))
 (segment (start 111 107.75) (end 111 122.25) (width 0.25) (layer F.Cu) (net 4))
 (segment (start 112.27 106.48) (end 111 107.75) (width 0.25) (layer F.Cu) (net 4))
 (segment (start 111 122.25) (end 111 122.25) (width 0.25) (layer F.Cu) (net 4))
 (via (at 111 122.25) (size 0.8) (drill 0.4) (layers F.Cu B.Cu) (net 4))
 (segment (start 113 122.25) (end 113 122.25) (width 0.25) (layer F.Cu) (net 2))
 (segment (start 114.73 109.02) (end 116.35 109.02) (width 0.25) (layer F.Cu) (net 2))
 (segment (start 113 110.75) (end 114.73 109.02) (width 0.25) (layer F.Cu) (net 2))
 (segment (start 113 122.25) (end 113 110.75) (width 0.25) (layer F.Cu) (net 2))
 (via (at 113 122.25) (size 0.8) (drill 0.4) (layers F.Cu B.Cu) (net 2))
 (segment (start 84 122.25) (end 84 122.25) (width 0.2) (layer F.Cu) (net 13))
 (segment (start 84 117.5) (end 85.75 115.75) (width 0.2) (layer F.Cu) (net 13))
 (segment (start 85.75 115.75) (end 85.75 108.75) (width 0.2) (layer F.Cu) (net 13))
 (segment (start 85.75 108.75) (end 86 108.5) (width 0.2) (layer F.Cu) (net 13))
 (segment (start 86 108.5) (end 86.25 108.5) (width 0.2) (layer F.Cu) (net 13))
 (segment (start 86.25 108.5) (end 86.784999 109.034999) (width 0.15) (layer F.Cu) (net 13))
 (segment (start 84 122.25) (end 84 117.5) (width 0.2) (layer F.Cu) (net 13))
 (via (at 84 122.25) (size 0.8) (drill 0.4) (layers F.Cu B.Cu) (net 13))
 (segment (start 103 122.25) (end 103 122.25) (width 0.5) (layer F.Cu) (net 5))
 (segment (start 103 116.75) (end 99.25 113) (width 0.5) (layer F.Cu) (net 5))
 (segment (start 99.25 113) (end 99.25 104.75) (width 0.5) (layer F.Cu) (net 5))
 (segment (start 100.06 103.94) (end 103.65 103.94) (width 0.5) (layer F.Cu) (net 5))
 (segment (start 99.25 104.75) (end 100.06 103.94) (width 0.5) (layer F.Cu) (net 5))
 (segment (start 103 122.25) (end 103 116.75) (width 0.5) (layer F.Cu) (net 5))
 (via (at 103 122.25) (size 0.8) (drill 0.4) (layers F.Cu B.Cu) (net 5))
 (segment (start 105 122.25) (end 105 122.25) (width 0.5) (layer F.Cu) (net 3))
 (segment (start 105 116.5) (end 100.75 112.25) (width 0.5) (layer F.Cu) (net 3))
 (segment (start 100.75 112.25) (end 100.75 105.875) (width 0.5) (layer F.Cu) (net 3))
 (segment (start 103.65 106.48) (end 103.17 106) (width 0.5) (layer F.Cu) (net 3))
 (segment (start 100.875 106) (end 100.75 105.875) (width 0.5) (layer F.Cu) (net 3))
 (segment (start 103.17 106) (end 100.875 106) (width 0.5) (layer F.Cu) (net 3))
 (segment (start 105 122.25) (end 105 116.5) (width 0.5) (layer F.Cu) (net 3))
 (via (at 105 122.25) (size 0.8) (drill 0.4) (layers F.Cu B.Cu) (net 3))
 (segment (start 115 122.25) (end 115 122.25) (width 0.25) (layer F.Cu) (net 1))
 (segment (start 115.94 111.56) (end 116.35 111.56) (width 0.25) (layer F.Cu) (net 1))
 (segment (start 115 112.5) (end 115.94 111.56) (width 0.25) (layer F.Cu) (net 1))
 (segment (start 115 122.25) (end 115 112.5) (width 0.25) (layer F.Cu) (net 1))
 (via (at 115 122.25) (size 0.8) (drill 0.4) (layers F.Cu B.Cu) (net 1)))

